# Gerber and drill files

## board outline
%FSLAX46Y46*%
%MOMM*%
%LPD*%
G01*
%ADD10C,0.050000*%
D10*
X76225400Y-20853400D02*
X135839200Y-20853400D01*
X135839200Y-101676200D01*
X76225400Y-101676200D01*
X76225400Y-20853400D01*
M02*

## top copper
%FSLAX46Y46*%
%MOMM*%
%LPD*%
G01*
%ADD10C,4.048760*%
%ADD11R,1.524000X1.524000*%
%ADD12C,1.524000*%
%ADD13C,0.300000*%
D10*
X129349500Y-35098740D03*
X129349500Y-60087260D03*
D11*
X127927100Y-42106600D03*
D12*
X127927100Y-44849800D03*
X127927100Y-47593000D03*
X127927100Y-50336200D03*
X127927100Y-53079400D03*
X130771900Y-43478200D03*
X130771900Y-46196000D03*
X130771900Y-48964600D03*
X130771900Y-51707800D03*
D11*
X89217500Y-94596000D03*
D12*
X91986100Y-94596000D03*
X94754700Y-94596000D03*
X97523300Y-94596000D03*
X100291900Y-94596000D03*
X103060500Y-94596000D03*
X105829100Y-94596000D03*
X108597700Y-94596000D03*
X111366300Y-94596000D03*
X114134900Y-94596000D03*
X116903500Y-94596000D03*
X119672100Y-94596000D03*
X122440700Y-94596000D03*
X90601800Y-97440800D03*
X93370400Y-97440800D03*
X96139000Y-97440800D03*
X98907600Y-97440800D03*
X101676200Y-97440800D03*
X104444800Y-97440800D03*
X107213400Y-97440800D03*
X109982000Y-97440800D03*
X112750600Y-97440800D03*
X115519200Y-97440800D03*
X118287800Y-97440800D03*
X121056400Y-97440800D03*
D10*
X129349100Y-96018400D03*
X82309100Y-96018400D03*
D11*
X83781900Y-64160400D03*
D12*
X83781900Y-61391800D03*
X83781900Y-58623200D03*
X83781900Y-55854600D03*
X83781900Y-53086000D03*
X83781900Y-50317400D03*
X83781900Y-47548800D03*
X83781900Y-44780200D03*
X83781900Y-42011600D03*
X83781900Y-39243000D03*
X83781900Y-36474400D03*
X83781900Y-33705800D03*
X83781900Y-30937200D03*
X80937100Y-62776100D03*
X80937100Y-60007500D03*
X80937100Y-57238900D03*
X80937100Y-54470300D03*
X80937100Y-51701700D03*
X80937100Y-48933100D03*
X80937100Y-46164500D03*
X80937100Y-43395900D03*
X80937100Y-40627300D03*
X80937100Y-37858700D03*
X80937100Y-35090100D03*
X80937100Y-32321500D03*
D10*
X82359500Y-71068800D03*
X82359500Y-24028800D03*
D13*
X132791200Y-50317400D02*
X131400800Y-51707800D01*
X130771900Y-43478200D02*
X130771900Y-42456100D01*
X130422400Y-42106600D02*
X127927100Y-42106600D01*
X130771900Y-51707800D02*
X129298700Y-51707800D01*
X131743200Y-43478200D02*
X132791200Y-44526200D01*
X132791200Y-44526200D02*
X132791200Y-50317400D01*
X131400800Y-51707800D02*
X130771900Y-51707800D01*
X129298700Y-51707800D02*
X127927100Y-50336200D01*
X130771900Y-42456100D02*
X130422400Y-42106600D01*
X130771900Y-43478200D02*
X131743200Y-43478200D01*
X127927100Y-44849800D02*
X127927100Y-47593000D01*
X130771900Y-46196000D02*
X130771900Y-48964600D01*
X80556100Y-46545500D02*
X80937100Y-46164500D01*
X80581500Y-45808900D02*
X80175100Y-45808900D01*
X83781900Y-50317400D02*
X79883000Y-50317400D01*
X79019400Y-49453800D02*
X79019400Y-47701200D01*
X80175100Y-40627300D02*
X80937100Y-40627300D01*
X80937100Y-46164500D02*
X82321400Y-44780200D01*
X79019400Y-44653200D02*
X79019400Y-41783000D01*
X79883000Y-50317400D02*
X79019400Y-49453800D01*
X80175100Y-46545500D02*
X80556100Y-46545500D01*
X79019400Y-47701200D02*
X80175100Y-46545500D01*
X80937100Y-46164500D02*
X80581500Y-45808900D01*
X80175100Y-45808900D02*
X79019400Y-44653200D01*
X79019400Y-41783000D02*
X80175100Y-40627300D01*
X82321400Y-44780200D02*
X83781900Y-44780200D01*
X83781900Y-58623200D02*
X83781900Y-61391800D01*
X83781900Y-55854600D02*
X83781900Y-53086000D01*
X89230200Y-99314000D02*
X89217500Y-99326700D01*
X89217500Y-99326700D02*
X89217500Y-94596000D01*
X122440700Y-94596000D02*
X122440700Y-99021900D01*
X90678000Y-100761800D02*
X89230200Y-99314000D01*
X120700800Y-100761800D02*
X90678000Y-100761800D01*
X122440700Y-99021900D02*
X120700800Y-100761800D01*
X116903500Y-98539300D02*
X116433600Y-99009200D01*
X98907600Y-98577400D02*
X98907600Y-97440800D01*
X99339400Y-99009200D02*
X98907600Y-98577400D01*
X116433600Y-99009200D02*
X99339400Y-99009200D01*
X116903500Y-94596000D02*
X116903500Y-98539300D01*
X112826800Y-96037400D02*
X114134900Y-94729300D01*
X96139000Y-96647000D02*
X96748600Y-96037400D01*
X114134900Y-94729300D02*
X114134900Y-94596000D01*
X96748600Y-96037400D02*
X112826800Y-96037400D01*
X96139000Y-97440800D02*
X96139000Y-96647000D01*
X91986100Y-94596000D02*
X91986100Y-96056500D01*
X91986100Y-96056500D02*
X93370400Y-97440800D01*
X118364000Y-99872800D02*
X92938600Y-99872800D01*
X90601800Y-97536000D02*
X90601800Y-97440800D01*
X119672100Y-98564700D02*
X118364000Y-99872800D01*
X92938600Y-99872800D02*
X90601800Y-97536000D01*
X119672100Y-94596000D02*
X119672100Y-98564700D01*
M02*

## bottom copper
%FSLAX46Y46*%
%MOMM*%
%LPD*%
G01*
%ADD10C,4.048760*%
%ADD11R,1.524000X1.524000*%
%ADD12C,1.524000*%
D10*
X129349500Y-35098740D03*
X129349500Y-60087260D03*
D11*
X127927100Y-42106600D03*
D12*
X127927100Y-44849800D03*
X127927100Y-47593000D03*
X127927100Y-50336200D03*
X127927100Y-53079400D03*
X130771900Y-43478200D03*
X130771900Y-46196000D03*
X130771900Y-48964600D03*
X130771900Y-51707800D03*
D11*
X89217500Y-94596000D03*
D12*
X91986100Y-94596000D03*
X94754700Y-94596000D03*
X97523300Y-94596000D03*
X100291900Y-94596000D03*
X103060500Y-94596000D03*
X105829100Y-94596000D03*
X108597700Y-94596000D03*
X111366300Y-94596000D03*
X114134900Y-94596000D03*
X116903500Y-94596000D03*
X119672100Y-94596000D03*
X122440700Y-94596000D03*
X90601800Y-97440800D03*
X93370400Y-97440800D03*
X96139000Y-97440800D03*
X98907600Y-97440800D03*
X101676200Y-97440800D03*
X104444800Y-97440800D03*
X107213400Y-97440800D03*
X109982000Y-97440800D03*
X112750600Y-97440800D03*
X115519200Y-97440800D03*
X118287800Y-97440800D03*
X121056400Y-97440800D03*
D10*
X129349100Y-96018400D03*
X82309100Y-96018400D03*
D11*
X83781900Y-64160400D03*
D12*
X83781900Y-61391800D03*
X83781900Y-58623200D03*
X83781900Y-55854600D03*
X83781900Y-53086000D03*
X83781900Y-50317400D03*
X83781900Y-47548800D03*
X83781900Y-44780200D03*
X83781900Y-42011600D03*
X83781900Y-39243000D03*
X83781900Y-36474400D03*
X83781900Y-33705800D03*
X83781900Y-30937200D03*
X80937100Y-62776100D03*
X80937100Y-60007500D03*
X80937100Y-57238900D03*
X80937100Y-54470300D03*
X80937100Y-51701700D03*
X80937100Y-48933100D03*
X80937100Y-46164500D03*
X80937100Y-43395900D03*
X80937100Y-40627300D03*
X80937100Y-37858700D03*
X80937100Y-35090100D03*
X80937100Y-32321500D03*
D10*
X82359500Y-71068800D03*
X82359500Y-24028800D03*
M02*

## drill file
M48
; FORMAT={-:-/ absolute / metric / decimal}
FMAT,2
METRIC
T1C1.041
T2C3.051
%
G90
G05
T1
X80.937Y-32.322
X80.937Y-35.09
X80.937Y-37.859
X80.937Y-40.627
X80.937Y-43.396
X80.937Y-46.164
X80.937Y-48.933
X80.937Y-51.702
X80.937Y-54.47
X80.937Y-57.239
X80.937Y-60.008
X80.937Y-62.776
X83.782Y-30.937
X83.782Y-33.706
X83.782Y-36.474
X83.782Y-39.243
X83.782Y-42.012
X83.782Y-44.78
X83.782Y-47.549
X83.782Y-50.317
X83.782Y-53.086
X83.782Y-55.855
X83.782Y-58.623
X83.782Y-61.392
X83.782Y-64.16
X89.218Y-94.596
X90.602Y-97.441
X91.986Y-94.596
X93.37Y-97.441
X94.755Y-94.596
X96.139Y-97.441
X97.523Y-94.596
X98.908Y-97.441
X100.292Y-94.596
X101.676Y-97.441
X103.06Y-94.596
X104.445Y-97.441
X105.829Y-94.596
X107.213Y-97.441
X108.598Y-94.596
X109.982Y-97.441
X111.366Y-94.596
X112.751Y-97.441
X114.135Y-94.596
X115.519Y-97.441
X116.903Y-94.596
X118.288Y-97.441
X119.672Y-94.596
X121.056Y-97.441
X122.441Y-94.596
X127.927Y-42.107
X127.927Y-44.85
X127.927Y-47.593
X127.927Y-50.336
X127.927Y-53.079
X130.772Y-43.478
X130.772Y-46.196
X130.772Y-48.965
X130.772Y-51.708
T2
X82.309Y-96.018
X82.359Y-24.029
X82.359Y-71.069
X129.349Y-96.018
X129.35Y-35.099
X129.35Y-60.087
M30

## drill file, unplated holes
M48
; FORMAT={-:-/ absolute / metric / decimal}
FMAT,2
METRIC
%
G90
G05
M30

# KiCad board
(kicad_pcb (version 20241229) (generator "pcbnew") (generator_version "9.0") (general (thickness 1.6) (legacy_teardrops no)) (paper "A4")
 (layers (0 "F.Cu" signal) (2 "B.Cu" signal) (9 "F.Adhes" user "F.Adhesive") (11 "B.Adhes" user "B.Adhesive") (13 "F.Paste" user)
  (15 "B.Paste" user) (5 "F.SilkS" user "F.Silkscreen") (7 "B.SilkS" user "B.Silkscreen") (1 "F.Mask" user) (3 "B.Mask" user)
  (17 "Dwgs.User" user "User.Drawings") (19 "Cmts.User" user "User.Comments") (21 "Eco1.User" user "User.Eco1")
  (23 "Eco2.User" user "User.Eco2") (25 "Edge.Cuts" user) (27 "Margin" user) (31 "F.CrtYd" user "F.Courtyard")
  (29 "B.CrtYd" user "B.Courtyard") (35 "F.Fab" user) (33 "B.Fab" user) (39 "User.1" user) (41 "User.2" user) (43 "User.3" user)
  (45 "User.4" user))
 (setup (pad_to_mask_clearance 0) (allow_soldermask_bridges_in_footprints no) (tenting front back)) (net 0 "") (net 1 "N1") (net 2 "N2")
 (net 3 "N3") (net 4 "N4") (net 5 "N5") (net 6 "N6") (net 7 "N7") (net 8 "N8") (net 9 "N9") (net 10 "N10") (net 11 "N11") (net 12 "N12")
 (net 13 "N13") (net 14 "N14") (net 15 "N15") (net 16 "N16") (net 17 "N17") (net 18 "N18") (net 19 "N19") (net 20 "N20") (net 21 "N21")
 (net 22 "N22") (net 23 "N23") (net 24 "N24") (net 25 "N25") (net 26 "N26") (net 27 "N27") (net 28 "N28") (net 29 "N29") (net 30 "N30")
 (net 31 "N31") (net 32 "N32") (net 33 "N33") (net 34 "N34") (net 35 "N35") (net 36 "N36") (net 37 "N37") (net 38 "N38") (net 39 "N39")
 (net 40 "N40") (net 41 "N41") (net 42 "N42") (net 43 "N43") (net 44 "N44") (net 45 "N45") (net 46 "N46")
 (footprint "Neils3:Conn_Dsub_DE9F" (layer "F.Cu") (at 129.3495 47.593 -90)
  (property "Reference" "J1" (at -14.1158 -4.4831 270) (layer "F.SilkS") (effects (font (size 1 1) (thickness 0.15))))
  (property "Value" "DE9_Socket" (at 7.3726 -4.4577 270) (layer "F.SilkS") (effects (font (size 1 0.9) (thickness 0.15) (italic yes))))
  (pad "0" thru_hole circle (at -12.49426 0 270) (size 4.04876 4.04876) (drill 3.05054) (layers "*.Cu" "*.Mask") (remove_unused_layers no)
   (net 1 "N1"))
  (pad "0" thru_hole circle (at 12.49426 0 270) (size 4.04876 4.04876) (drill 3.05054) (layers "*.Cu" "*.Mask") (remove_unused_layers no)
   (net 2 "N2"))
  (pad "1" thru_hole rect (at -5.4864 1.4224 270) (size 1.524 1.524) (drill 1.0414) (layers "*.Cu" "*.Mask") (remove_unused_layers no)
   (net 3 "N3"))
  (pad "2" thru_hole circle (at -2.7432 1.4224 270) (size 1.524 1.524) (drill 1.0414) (layers "*.Cu" "*.Mask") (remove_unused_layers no)
   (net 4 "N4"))
  (pad "3" thru_hole circle (at 0 1.4224 270) (size 1.524 1.524) (drill 1.0414) (layers "*.Cu" "*.Mask") (remove_unused_layers no)
   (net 4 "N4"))
  (pad "4" thru_hole circle (at 2.7432 1.4224 270) (size 1.524 1.524) (drill 1.0414) (layers "*.Cu" "*.Mask") (remove_unused_layers no)
   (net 3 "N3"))
  (pad "5" thru_hole circle (at 5.4864 1.4224 270) (size 1.524 1.524) (drill 1.0414) (layers "*.Cu" "*.Mask") (remove_unused_layers no)
   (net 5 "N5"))
  (pad "6" thru_hole circle (at -4.1148 -1.4224 270) (size 1.524 1.524) (drill 1.0414) (layers "*.Cu" "*.Mask") (remove_unused_layers no)
   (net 3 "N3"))
  (pad "7" thru_hole circle (at -1.397 -1.4224 270) (size 1.524 1.524) (drill 1.0414) (layers "*.Cu" "*.Mask") (remove_unused_layers no)
   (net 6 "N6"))
  (pad "8" thru_hole circle (at 1.3716 -1.4224 270) (size 1.524 1.524) (drill 1.0414) (layers "*.Cu" "*.Mask") (remove_unused_layers no)
   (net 6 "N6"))
  (pad "9" thru_hole circle (at 4.1148 -1.4224 270) (size 1.524 1.524) (drill 1.0414) (layers "*.Cu" "*.Mask") (remove_unused_layers no)
   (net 3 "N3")))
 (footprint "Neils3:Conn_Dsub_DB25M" (layer "F.Cu") (at 105.8291 96.0184 180)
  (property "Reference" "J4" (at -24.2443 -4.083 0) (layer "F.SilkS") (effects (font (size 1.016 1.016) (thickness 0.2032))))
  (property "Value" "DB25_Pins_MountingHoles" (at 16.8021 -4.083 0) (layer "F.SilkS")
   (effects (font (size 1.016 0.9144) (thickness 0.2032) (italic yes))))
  (pad "1" thru_hole rect (at 16.6116 1.4224 180) (size 1.524 1.524) (drill 1.0414) (layers "*.Cu" "*.Mask" "F.SilkS")
   (remove_unused_layers no) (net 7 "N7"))
  (pad "2" thru_hole circle (at 13.843 1.4224 180) (size 1.524 1.524) (drill 1.0414) (layers "*.Cu" "*.Mask" "F.SilkS")
   (remove_unused_layers no) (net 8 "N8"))
  (pad "3" thru_hole circle (at 11.0744 1.4224 180) (size 1.524 1.524) (drill 1.0414) (layers "*.Cu" "*.Mask" "F.SilkS")
   (remove_unused_layers no) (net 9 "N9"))
  (pad "4" thru_hole circle (at 8.3058 1.4224 180) (size 1.524 1.524) (drill 1.0414) (layers "*.Cu" "*.Mask" "F.SilkS")
   (remove_unused_layers no) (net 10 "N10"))
  (pad "5" thru_hole circle (at 5.5372 1.4224 180) (size 1.524 1.524) (drill 1.0414) (layers "*.Cu" "*.Mask" "F.SilkS")
   (remove_unused_layers no) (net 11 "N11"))
  (pad "6" thru_hole circle (at 2.7686 1.4224 180) (size 1.524 1.524) (drill 1.0414) (layers "*.Cu" "*.Mask" "F.SilkS")
   (remove_unused_layers no) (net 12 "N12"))
  (pad "7" thru_hole circle (at 0 1.4224 180) (size 1.524 1.524) (drill 1.0414) (layers "*.Cu" "*.Mask" "F.SilkS") (remove_unused_layers no)
   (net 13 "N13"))
  (pad "8" thru_hole circle (at -2.7686 1.4224 180) (size 1.524 1.524) (drill 1.0414) (layers "*.Cu" "*.Mask" "F.SilkS")
   (remove_unused_layers no) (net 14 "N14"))
  (pad "9" thru_hole circle (at -5.5372 1.4224 180) (size 1.524 1.524) (drill 1.0414) (layers "*.Cu" "*.Mask" "F.SilkS")
   (remove_unused_layers no) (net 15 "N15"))
  (pad "10" thru_hole circle (at -8.3058 1.4224 180) (size 1.524 1.524) (drill 1.0414) (layers "*.Cu" "*.Mask" "F.SilkS")
   (remove_unused_layers no) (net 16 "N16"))
  (pad "11" thru_hole circle (at -11.0744 1.4224 180) (size 1.524 1.524) (drill 1.0414) (layers "*.Cu" "*.Mask" "F.SilkS")
   (remove_unused_layers no) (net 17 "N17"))
  (pad "12" thru_hole circle (at -13.843 1.4224 180) (size 1.524 1.524) (drill 1.0414) (layers "*.Cu" "*.Mask" "F.SilkS")
   (remove_unused_layers no) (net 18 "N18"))
  (pad "13" thru_hole circle (at -16.6116 1.4224 180) (size 1.524 1.524) (drill 1.0414) (layers "*.Cu" "*.Mask" "F.SilkS")
   (remove_unused_layers no) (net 7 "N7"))
  (pad "14" thru_hole circle (at 15.2273 -1.4224 180) (size 1.524 1.524) (drill 1.0414) (layers "*.Cu" "*.Mask" "F.SilkS")
   (remove_unused_layers no) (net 18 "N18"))
  (pad "15" thru_hole circle (at 12.4587 -1.4224 180) (size 1.524 1.524) (drill 1.0414) (layers "*.Cu" "*.Mask" "F.SilkS")
   (remove_unused_layers no) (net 8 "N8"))
  (pad "16" thru_hole circle (at 9.6901 -1.4224 180) (size 1.524 1.524) (drill 1.0414) (layers "*.Cu" "*.Mask" "F.SilkS")
   (remove_unused_layers no) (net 16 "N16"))
  (pad "17" thru_hole circle (at 6.9215 -1.4224 180) (size 1.524 1.524) (drill 1.0414) (layers "*.Cu" "*.Mask" "F.SilkS")
   (remove_unused_layers no) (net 17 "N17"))
  (pad "18" thru_hole circle (at 4.1529 -1.4224 180) (size 1.524 1.524) (drill 1.0414) (layers "*.Cu" "*.Mask" "F.SilkS")
   (remove_unused_layers no) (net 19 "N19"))
  (pad "19" thru_hole circle (at 1.3843 -1.4224 180) (size 1.524 1.524) (drill 1.0414) (layers "*.Cu" "*.Mask" "F.SilkS")
   (remove_unused_layers no) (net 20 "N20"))
  (pad "20" thru_hole circle (at -1.3843 -1.4224 180) (size 1.524 1.524) (drill 1.0414) (layers "*.Cu" "*.Mask" "F.SilkS")
   (remove_unused_layers no) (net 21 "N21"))
  (pad "21" thru_hole circle (at -4.1529 -1.4224 180) (size 1.524 1.524) (drill 1.0414) (layers "*.Cu" "*.Mask" "F.SilkS")
   (remove_unused_layers no) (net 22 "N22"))
  (pad "22" thru_hole circle (at -6.9215 -1.4224 180) (size 1.524 1.524) (drill 1.0414) (layers "*.Cu" "*.Mask" "F.SilkS")
   (remove_unused_layers no) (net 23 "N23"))
  (pad "23" thru_hole circle (at -9.6901 -1.4224 180) (size 1.524 1.524) (drill 1.0414) (layers "*.Cu" "*.Mask" "F.SilkS")
   (remove_unused_layers no) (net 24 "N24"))
  (pad "24" thru_hole circle (at -12.4587 -1.4224 180) (size 1.524 1.524) (drill 1.0414) (layers "*.Cu" "*.Mask" "F.SilkS")
   (remove_unused_layers no) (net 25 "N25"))
  (pad "25" thru_hole circle (at -15.2273 -1.4224 180) (size 1.524 1.524) (drill 1.0414) (layers "*.Cu" "*.Mask" "F.SilkS")
   (remove_unused_layers no) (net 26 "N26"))
  (pad "GND" thru_hole circle (at -23.52 0 180) (size 4.04876 4.04876) (drill 3.05054) (layers "*.Cu" "*.Mask" "F.SilkS")
   (remove_unused_layers no))
  (pad "GND" thru_hole circle (at 23.52 0 180) (size 4.04876 4.04876) (drill 3.05054) (layers "*.Cu" "*.Mask" "F.SilkS")
   (remove_unused_layers no)))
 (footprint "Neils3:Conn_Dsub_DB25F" (layer "F.Cu") (at 82.3595 47.5488 90)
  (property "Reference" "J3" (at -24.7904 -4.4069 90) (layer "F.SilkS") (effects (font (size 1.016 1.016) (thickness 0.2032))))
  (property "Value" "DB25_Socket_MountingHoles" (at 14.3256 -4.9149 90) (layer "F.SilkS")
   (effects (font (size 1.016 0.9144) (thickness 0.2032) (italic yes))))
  (pad "1" thru_hole rect (at -16.6116 1.4224 90) (size 1.524 1.524) (drill 1.0414) (layers "*.Cu" "*.Mask" "F.SilkS")
   (remove_unused_layers no) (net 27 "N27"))
  (pad "2" thru_hole circle (at -13.843 1.4224 90) (size 1.524 1.524) (drill 1.0414) (layers "*.Cu" "*.Mask" "F.SilkS")
   (remove_unused_layers no) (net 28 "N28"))
  (pad "3" thru_hole circle (at -11.0744 1.4224 90) (size 1.524 1.524) (drill 1.0414) (layers "*.Cu" "*.Mask" "F.SilkS")
   (remove_unused_layers no) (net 28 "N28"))
  (pad "4" thru_hole circle (at -8.3058 1.4224 90) (size 1.524 1.524) (drill 1.0414) (layers "*.Cu" "*.Mask" "F.SilkS")
   (remove_unused_layers no) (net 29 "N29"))
  (pad "5" thru_hole circle (at -5.5372 1.4224 90) (size 1.524 1.524) (drill 1.0414) (layers "*.Cu" "*.Mask" "F.SilkS")
   (remove_unused_layers no) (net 29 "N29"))
  (pad "6" thru_hole circle (at -2.7686 1.4224 90) (size 1.524 1.524) (drill 1.0414) (layers "*.Cu" "*.Mask" "F.SilkS")
   (remove_unused_layers no) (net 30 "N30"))
  (pad "7" thru_hole circle (at 0 1.4224 90) (size 1.524 1.524) (drill 1.0414) (layers "*.Cu" "*.Mask" "F.SilkS") (remove_unused_layers no)
   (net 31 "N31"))
  (pad "8" thru_hole circle (at 2.7686 1.4224 90) (size 1.524 1.524) (drill 1.0414) (layers "*.Cu" "*.Mask" "F.SilkS")
   (remove_unused_layers no) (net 30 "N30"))
  (pad "9" thru_hole circle (at 5.5372 1.4224 90) (size 1.524 1.524) (drill 1.0414) (layers "*.Cu" "*.Mask" "F.SilkS")
   (remove_unused_layers no) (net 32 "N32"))
  (pad "10" thru_hole circle (at 8.3058 1.4224 90) (size 1.524 1.524) (drill 1.0414) (layers "*.Cu" "*.Mask" "F.SilkS")
   (remove_unused_layers no) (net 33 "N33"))
  (pad "11" thru_hole circle (at 11.0744 1.4224 90) (size 1.524 1.524) (drill 1.0414) (layers "*.Cu" "*.Mask" "F.SilkS")
   (remove_unused_layers no) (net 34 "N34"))
  (pad "12" thru_hole circle (at 13.843 1.4224 90) (size 1.524 1.524) (drill 1.0414) (layers "*.Cu" "*.Mask" "F.SilkS")
   (remove_unused_layers no) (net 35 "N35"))
  (pad "13" thru_hole circle (at 16.6116 1.4224 90) (size 1.524 1.524) (drill 1.0414) (layers "*.Cu" "*.Mask" "F.SilkS")
   (remove_unused_layers no) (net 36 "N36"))
  (pad "14" thru_hole circle (at -15.2273 -1.4224 90) (size 1.524 1.524) (drill 1.0414) (layers "*.Cu" "*.Mask" "F.SilkS")
   (remove_unused_layers no) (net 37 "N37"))
  (pad "15" thru_hole circle (at -12.4587 -1.4224 90) (size 1.524 1.524) (drill 1.0414) (layers "*.Cu" "*.Mask" "F.SilkS")
   (remove_unused_layers no) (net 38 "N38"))
  (pad "16" thru_hole circle (at -9.6901 -1.4224 90) (size 1.524 1.524) (drill 1.0414) (layers "*.Cu" "*.Mask" "F.SilkS")
   (remove_unused_layers no) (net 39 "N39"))
  (pad "17" thru_hole circle (at -6.9215 -1.4224 90) (size 1.524 1.524) (drill 1.0414) (layers "*.Cu" "*.Mask" "F.SilkS")
   (remove_unused_layers no) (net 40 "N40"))
  (pad "18" thru_hole circle (at -4.1529 -1.4224 90) (size 1.524 1.524) (drill 1.0414) (layers "*.Cu" "*.Mask" "F.SilkS")
   (remove_unused_layers no) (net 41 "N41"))
  (pad "19" thru_hole circle (at -1.3843 -1.4224 90) (size 1.524 1.524) (drill 1.0414) (layers "*.Cu" "*.Mask" "F.SilkS")
   (remove_unused_layers no) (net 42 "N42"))
  (pad "20" thru_hole circle (at 1.3843 -1.4224 90) (size 1.524 1.524) (drill 1.0414) (layers "*.Cu" "*.Mask" "F.SilkS")
   (remove_unused_layers no) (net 30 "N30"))
  (pad "21" thru_hole circle (at 4.1529 -1.4224 90) (size 1.524 1.524) (drill 1.0414) (layers "*.Cu" "*.Mask" "F.SilkS")
   (remove_unused_layers no) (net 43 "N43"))
  (pad "22" thru_hole circle (at 6.9215 -1.4224 90) (size 1.524 1.524) (drill 1.0414) (layers "*.Cu" "*.Mask" "F.SilkS")
   (remove_unused_layers no) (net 30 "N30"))
  (pad "23" thru_hole circle (at 9.6901 -1.4224 90) (size 1.524 1.524) (drill 1.0414) (layers "*.Cu" "*.Mask" "F.SilkS")
   (remove_unused_layers no) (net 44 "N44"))
  (pad "24" thru_hole circle (at 12.4587 -1.4224 90) (size 1.524 1.524) (drill 1.0414) (layers "*.Cu" "*.Mask" "F.SilkS")
   (remove_unused_layers no) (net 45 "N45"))
  (pad "25" thru_hole circle (at 15.2273 -1.4224 90) (size 1.524 1.524) (drill 1.0414) (layers "*.Cu" "*.Mask" "F.SilkS")
   (remove_unused_layers no) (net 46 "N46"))
  (pad "GND" thru_hole circle (at -23.52 0 90) (size 4.04876 4.04876) (drill 3.05054) (layers "*.Cu" "*.Mask" "F.SilkS")
   (remove_unused_layers no))
  (pad "GND" thru_hole circle (at 23.52 0 90) (size 4.04876 4.04876) (drill 3.05054) (layers "*.Cu" "*.Mask" "F.SilkS")
   (remove_unused_layers no)))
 (gr_rect (start 76.2254 20.8534) (end 135.8392 101.6762) (stroke (width 0.05) (type default)) (fill no) (layer "Edge.Cuts"))
 (segment (start 132.7912 50.3174) (end 131.4008 51.7078) (width 0.3) (layer "F.Cu") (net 3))
 (segment (start 130.7719 43.4782) (end 130.7719 42.4561) (width 0.3) (layer "F.Cu") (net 3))
 (segment (start 130.4224 42.1066) (end 127.9271 42.1066) (width 0.3) (layer "F.Cu") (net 3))
 (segment (start 130.7719 51.7078) (end 129.2987 51.7078) (width 0.3) (layer "F.Cu") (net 3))
 (segment (start 131.7432 43.4782) (end 132.7912 44.5262) (width 0.3) (layer "F.Cu") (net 3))
 (segment (start 132.7912 44.5262) (end 132.7912 50.3174) (width 0.3) (layer "F.Cu") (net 3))
 (segment (start 131.4008 51.7078) (end 130.7719 51.7078) (width 0.3) (layer "F.Cu") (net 3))
 (segment (start 129.2987 51.7078) (end 127.9271 50.3362) (width 0.3) (layer "F.Cu") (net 3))
 (segment (start 130.7719 42.4561) (end 130.4224 42.1066) (width 0.3) (layer "F.Cu") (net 3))
 (segment (start 130.7719 43.4782) (end 131.7432 43.4782) (width 0.3) (layer "F.Cu") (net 3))
 (segment (start 127.9271 44.8498) (end 127.9271 47.593) (width 0.3) (layer "F.Cu") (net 4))
 (segment (start 130.7719 46.196) (end 130.7719 48.9646) (width 0.3) (layer "F.Cu") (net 6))
 (segment (start 80.5561 46.5455) (end 80.9371 46.1645) (width 0.3) (layer "F.Cu") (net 30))
 (segment (start 80.5815 45.8089) (end 80.1751 45.8089) (width 0.3) (layer "F.Cu") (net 30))
 (segment (start 83.7819 50.3174) (end 79.883 50.3174) (width 0.3) (layer "F.Cu") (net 30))
 (segment (start 79.0194 49.4538) (end 79.0194 47.7012) (width 0.3) (layer "F.Cu") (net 30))
 (segment (start 80.1751 40.6273) (end 80.9371 40.6273) (width 0.3) (layer "F.Cu") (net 30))
 (segment (start 80.9371 46.1645) (end 82.3214 44.7802) (width 0.3) (layer "F.Cu") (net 30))
 (segment (start 79.0194 44.6532) (end 79.0194 41.783) (width 0.3) (layer "F.Cu") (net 30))
 (segment (start 79.883 50.3174) (end 79.0194 49.4538) (width 0.3) (layer "F.Cu") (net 30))
 (segment (start 80.1751 46.5455) (end 80.5561 46.5455) (width 0.3) (layer "F.Cu") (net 30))
 (segment (start 79.0194 47.7012) (end 80.1751 46.5455) (width 0.3) (layer "F.Cu") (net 30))
 (segment (start 80.9371 46.1645) (end 80.5815 45.8089) (width 0.3) (layer "F.Cu") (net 30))
 (segment (start 80.1751 45.8089) (end 79.0194 44.6532) (width 0.3) (layer "F.Cu") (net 30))
 (segment (start 79.0194 41.783) (end 80.1751 40.6273) (width 0.3) (layer "F.Cu") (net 30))
 (segment (start 82.3214 44.7802) (end 83.7819 44.7802) (width 0.3) (layer "F.Cu") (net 30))
 (segment (start 83.7819 58.6232) (end 83.7819 61.3918) (width 0.3) (layer "F.Cu") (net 28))
 (segment (start 83.7819 55.8546) (end 83.7819 53.086) (width 0.3) (layer "F.Cu") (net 29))
 (segment (start 89.2302 99.314) (end 89.2175 99.3267) (width 0.3) (layer "F.Cu") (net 7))
 (segment (start 89.2175 99.3267) (end 89.2175 94.596) (width 0.3) (layer "F.Cu") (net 7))
 (segment (start 122.4407 94.596) (end 122.4407 99.0219) (width 0.3) (layer "F.Cu") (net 7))
 (segment (start 90.678 100.7618) (end 89.2302 99.314) (width 0.3) (layer "F.Cu") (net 7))
 (segment (start 120.7008 100.7618) (end 90.678 100.7618) (width 0.3) (layer "F.Cu") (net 7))
 (segment (start 122.4407 99.0219) (end 120.7008 100.7618) (width 0.3) (layer "F.Cu") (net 7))
 (segment (start 116.9035 98.5393) (end 116.4336 99.0092) (width 0.3) (layer "F.Cu") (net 17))
 (segment (start 98.9076 98.5774) (end 98.9076 97.4408) (width 0.3) (layer "F.Cu") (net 17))
 (segment (start 99.3394 99.0092) (end 98.9076 98.5774) (width 0.3) (layer "F.Cu") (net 17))
 (segment (start 116.4336 99.0092) (end 99.3394 99.0092) (width 0.3) (layer "F.Cu") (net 17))
 (segment (start 116.9035 94.596) (end 116.9035 98.5393) (width 0.3) (layer "F.Cu") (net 17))
 (segment (start 112.8268 96.0374) (end 114.1349 94.7293) (width 0.3) (layer "F.Cu") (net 16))
 (segment (start 96.139 96.647) (end 96.7486 96.0374) (width 0.3) (layer "F.Cu") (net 16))
 (segment (start 114.1349 94.7293) (end 114.1349 94.596) (width 0.3) (layer "F.Cu") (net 16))
 (segment (start 96.7486 96.0374) (end 112.8268 96.0374) (width 0.3) (layer "F.Cu") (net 16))
 (segment (start 96.139 97.4408) (end 96.139 96.647) (width 0.3) (layer "F.Cu") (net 16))
 (segment (start 91.9861 94.596) (end 91.9861 96.0565) (width 0.3) (layer "F.Cu") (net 8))
 (segment (start 91.9861 96.0565) (end 93.3704 97.4408) (width 0.3) (layer "F.Cu") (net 8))
 (segment (start 118.364 99.8728) (end 92.9386 99.8728) (width 0.3) (layer "F.Cu") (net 18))
 (segment (start 90.6018 97.536) (end 90.6018 97.4408) (width 0.3) (layer "F.Cu") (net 18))
 (segment (start 119.6721 98.5647) (end 118.364 99.8728) (width 0.3) (layer "F.Cu") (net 18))
 (segment (start 92.9386 99.8728) (end 90.6018 97.536) (width 0.3) (layer "F.Cu") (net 18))
 (segment (start 119.6721 94.596) (end 119.6721 98.5647) (width 0.3) (layer "F.Cu") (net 18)))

